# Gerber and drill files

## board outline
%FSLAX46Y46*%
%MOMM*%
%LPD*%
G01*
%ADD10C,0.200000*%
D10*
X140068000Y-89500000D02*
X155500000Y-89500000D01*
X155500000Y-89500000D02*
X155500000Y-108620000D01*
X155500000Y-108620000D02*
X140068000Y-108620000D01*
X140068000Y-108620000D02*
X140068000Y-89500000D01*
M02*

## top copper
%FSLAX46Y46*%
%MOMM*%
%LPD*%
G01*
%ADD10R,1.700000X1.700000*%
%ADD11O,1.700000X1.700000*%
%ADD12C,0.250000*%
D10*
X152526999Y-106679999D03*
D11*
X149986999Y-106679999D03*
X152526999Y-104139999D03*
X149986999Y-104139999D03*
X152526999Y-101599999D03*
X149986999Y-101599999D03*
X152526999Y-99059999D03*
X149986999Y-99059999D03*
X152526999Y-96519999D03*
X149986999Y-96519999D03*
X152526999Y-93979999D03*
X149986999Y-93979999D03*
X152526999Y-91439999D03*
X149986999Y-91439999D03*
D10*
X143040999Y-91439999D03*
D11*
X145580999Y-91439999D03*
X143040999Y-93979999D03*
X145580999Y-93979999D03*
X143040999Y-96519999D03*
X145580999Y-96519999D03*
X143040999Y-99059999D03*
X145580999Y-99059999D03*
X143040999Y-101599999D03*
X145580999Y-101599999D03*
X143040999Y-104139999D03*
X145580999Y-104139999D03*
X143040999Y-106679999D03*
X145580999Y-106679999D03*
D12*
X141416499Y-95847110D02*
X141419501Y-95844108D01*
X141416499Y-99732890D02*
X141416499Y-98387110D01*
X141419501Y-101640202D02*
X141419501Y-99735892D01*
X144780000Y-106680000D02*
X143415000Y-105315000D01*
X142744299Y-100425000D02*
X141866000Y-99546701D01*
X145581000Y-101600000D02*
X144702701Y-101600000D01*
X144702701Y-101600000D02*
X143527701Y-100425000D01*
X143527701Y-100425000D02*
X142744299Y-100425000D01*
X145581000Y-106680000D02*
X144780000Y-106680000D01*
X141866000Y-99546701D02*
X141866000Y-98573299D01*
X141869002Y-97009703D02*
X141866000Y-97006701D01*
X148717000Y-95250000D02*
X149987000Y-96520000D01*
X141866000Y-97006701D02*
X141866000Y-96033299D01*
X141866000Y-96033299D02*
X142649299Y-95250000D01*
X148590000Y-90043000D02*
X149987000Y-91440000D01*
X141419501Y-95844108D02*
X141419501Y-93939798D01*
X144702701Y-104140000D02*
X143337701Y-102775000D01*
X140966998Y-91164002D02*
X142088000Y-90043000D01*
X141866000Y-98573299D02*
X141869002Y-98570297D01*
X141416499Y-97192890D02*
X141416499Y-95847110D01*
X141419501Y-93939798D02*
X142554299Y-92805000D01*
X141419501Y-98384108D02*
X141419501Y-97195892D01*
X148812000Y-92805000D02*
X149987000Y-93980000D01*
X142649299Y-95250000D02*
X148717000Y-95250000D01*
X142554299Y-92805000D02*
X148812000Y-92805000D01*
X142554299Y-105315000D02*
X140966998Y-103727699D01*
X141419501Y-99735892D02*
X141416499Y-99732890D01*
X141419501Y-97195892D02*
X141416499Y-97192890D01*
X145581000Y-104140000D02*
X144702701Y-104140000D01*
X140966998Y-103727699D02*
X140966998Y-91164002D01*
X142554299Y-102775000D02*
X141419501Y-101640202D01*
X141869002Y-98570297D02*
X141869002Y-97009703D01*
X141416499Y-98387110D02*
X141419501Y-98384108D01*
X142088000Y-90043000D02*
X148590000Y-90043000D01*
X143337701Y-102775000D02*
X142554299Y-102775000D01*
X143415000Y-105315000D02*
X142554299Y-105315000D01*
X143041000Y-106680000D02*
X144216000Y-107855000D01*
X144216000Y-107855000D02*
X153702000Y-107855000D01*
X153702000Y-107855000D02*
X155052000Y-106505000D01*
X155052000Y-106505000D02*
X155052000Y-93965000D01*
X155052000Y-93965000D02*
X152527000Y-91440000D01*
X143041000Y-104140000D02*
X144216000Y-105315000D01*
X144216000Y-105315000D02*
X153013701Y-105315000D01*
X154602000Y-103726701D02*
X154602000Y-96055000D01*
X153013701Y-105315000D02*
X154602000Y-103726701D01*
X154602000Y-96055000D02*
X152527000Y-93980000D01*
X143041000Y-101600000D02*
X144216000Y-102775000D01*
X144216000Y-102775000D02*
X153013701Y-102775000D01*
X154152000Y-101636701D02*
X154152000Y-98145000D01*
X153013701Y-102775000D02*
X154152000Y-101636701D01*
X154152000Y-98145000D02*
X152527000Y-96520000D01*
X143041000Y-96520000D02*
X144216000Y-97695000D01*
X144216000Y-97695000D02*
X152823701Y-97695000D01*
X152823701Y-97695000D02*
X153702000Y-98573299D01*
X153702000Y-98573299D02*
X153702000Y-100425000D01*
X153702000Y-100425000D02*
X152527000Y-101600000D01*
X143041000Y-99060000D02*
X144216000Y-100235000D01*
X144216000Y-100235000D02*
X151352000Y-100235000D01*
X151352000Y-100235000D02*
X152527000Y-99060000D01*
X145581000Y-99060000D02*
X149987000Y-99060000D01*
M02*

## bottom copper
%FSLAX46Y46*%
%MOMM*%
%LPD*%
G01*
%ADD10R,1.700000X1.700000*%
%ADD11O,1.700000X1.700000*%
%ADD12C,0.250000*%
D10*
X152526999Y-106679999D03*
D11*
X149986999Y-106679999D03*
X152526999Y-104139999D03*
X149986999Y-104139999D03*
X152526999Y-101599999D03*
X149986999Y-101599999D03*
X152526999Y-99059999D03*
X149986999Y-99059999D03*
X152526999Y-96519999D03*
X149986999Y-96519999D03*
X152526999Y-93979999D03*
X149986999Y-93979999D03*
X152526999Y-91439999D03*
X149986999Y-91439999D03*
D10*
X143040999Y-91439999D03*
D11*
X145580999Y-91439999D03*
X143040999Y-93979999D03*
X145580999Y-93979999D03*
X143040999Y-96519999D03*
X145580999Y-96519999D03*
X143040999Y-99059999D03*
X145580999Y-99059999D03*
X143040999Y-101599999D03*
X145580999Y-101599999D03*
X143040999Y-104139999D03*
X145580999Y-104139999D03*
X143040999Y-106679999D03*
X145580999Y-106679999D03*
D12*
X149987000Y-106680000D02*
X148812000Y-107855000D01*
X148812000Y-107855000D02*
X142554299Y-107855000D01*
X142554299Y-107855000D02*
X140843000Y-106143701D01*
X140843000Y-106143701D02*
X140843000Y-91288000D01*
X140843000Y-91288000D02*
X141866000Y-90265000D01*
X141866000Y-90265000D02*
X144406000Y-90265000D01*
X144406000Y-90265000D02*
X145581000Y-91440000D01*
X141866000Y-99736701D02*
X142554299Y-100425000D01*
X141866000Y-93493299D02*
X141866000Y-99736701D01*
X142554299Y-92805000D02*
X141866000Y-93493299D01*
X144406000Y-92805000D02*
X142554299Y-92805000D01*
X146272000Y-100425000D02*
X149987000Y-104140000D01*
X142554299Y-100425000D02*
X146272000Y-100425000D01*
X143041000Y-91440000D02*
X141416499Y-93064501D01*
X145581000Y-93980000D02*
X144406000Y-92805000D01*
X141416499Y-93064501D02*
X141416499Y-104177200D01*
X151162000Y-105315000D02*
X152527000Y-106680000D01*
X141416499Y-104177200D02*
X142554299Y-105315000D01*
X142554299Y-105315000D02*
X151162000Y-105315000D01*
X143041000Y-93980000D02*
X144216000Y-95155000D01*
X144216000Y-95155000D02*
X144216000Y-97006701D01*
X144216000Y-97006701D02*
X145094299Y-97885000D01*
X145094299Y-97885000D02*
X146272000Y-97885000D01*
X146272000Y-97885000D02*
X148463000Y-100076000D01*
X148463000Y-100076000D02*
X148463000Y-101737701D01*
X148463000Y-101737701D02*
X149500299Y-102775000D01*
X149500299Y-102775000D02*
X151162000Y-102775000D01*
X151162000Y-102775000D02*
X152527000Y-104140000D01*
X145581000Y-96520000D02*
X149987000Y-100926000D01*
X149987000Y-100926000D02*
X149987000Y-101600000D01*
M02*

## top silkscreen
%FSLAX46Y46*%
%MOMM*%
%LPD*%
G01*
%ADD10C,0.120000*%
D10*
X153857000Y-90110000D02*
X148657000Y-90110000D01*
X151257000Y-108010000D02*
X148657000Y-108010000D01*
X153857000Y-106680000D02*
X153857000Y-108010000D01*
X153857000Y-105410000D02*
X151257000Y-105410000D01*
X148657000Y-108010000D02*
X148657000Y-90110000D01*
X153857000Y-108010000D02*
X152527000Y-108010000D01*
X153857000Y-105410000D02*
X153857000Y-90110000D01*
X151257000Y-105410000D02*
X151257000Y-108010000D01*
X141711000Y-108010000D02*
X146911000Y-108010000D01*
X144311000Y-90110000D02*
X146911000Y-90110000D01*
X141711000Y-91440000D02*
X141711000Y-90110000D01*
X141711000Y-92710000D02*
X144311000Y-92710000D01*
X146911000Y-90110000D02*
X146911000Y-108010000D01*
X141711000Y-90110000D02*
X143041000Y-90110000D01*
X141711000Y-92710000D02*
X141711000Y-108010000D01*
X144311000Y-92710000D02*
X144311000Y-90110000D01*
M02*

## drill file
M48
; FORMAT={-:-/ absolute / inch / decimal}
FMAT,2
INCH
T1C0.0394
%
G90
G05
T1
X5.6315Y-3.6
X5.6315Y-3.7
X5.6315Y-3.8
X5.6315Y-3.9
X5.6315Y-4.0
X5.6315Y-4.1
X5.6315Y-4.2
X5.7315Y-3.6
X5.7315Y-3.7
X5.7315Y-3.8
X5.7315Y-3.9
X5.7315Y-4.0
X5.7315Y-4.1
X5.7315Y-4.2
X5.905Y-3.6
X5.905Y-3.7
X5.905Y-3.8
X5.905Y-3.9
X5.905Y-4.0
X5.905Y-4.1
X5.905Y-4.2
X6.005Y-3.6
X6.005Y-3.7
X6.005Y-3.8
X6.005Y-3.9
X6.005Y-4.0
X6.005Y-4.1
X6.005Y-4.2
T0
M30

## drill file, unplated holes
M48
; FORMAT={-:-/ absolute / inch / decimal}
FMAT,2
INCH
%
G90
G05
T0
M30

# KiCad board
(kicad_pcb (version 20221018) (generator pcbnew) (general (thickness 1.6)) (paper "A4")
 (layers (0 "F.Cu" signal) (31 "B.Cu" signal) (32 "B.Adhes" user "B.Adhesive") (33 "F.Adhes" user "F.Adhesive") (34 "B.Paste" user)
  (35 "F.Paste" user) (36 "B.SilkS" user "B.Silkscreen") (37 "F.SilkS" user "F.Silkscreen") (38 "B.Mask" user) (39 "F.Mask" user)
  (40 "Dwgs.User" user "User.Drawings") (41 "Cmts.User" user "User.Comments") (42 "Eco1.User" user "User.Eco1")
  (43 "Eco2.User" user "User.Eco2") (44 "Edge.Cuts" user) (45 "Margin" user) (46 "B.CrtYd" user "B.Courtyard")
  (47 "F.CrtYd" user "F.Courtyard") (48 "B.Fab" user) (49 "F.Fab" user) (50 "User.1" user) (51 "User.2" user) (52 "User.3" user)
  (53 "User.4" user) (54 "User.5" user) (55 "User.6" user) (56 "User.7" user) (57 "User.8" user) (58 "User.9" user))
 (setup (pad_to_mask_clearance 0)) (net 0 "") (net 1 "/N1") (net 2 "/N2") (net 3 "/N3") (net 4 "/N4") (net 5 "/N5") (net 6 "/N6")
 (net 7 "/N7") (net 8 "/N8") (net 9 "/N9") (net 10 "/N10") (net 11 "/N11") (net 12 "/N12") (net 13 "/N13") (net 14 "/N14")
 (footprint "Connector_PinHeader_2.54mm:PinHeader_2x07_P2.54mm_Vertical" (layer "F.Cu") (at 143.041 91.44)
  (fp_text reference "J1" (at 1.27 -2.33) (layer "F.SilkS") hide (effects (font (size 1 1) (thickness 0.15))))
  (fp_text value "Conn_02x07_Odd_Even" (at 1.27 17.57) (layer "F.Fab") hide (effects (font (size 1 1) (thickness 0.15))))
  (fp_line (start -1.33 -1.33) (end 0 -1.33) (stroke (width 0.12) (type solid)) (layer "F.SilkS"))
  (fp_line (start -1.33 0) (end -1.33 -1.33) (stroke (width 0.12) (type solid)) (layer "F.SilkS"))
  (fp_line (start -1.33 1.27) (end -1.33 16.57) (stroke (width 0.12) (type solid)) (layer "F.SilkS"))
  (fp_line (start -1.33 1.27) (end 1.27 1.27) (stroke (width 0.12) (type solid)) (layer "F.SilkS"))
  (fp_line (start -1.33 16.57) (end 3.87 16.57) (stroke (width 0.12) (type solid)) (layer "F.SilkS"))
  (fp_line (start 1.27 -1.33) (end 3.87 -1.33) (stroke (width 0.12) (type solid)) (layer "F.SilkS"))
  (fp_line (start 1.27 1.27) (end 1.27 -1.33) (stroke (width 0.12) (type solid)) (layer "F.SilkS"))
  (fp_line (start 3.87 -1.33) (end 3.87 16.57) (stroke (width 0.12) (type solid)) (layer "F.SilkS"))
  (pad "1" thru_hole rect (at 0 0) (size 1.7 1.7) (drill 1) (layers "*.Cu" "*.Mask") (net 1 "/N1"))
  (pad "2" thru_hole oval (at 2.54 0) (size 1.7 1.7) (drill 1) (layers "*.Cu" "*.Mask") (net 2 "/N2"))
  (pad "3" thru_hole oval (at 0 2.54) (size 1.7 1.7) (drill 1) (layers "*.Cu" "*.Mask") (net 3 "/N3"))
  (pad "4" thru_hole oval (at 2.54 2.54) (size 1.7 1.7) (drill 1) (layers "*.Cu" "*.Mask") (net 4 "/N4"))
  (pad "5" thru_hole oval (at 0 5.08) (size 1.7 1.7) (drill 1) (layers "*.Cu" "*.Mask") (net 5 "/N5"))
  (pad "6" thru_hole oval (at 2.54 5.08) (size 1.7 1.7) (drill 1) (layers "*.Cu" "*.Mask") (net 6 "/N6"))
  (pad "7" thru_hole oval (at 0 7.62) (size 1.7 1.7) (drill 1) (layers "*.Cu" "*.Mask") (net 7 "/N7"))
  (pad "8" thru_hole oval (at 2.54 7.62) (size 1.7 1.7) (drill 1) (layers "*.Cu" "*.Mask") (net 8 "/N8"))
  (pad "9" thru_hole oval (at 0 10.16) (size 1.7 1.7) (drill 1) (layers "*.Cu" "*.Mask") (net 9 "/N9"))
  (pad "10" thru_hole oval (at 2.54 10.16) (size 1.7 1.7) (drill 1) (layers "*.Cu" "*.Mask") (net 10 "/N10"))
  (pad "11" thru_hole oval (at 0 12.7) (size 1.7 1.7) (drill 1) (layers "*.Cu" "*.Mask") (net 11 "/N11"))
  (pad "12" thru_hole oval (at 2.54 12.7) (size 1.7 1.7) (drill 1) (layers "*.Cu" "*.Mask") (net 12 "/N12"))
  (pad "13" thru_hole oval (at 0 15.24) (size 1.7 1.7) (drill 1) (layers "*.Cu" "*.Mask") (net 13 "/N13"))
  (pad "14" thru_hole oval (at 2.54 15.24) (size 1.7 1.7) (drill 1) (layers "*.Cu" "*.Mask") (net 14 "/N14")))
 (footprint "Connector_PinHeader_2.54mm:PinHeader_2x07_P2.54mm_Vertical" (layer "F.Cu") (at 152.527 106.68 180)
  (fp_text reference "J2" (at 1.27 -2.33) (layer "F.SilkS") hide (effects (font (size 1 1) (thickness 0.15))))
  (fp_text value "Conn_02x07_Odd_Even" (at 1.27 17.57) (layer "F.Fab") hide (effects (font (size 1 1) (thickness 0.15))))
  (fp_line (start -1.33 -1.33) (end 0 -1.33) (stroke (width 0.12) (type solid)) (layer "F.SilkS"))
  (fp_line (start -1.33 0) (end -1.33 -1.33) (stroke (width 0.12) (type solid)) (layer "F.SilkS"))
  (fp_line (start -1.33 1.27) (end -1.33 16.57) (stroke (width 0.12) (type solid)) (layer "F.SilkS"))
  (fp_line (start -1.33 1.27) (end 1.27 1.27) (stroke (width 0.12) (type solid)) (layer "F.SilkS"))
  (fp_line (start -1.33 16.57) (end 3.87 16.57) (stroke (width 0.12) (type solid)) (layer "F.SilkS"))
  (fp_line (start 1.27 -1.33) (end 3.87 -1.33) (stroke (width 0.12) (type solid)) (layer "F.SilkS"))
  (fp_line (start 1.27 1.27) (end 1.27 -1.33) (stroke (width 0.12) (type solid)) (layer "F.SilkS"))
  (fp_line (start 3.87 -1.33) (end 3.87 16.57) (stroke (width 0.12) (type solid)) (layer "F.SilkS"))
  (pad "1" thru_hole rect (at 0 0 180) (size 1.7 1.7) (drill 1) (layers "*.Cu" "*.Mask") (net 1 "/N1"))
  (pad "2" thru_hole oval (at 2.54 0 180) (size 1.7 1.7) (drill 1) (layers "*.Cu" "*.Mask") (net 2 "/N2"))
  (pad "3" thru_hole oval (at 0 2.54 180) (size 1.7 1.7) (drill 1) (layers "*.Cu" "*.Mask") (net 3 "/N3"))
  (pad "4" thru_hole oval (at 2.54 2.54 180) (size 1.7 1.7) (drill 1) (layers "*.Cu" "*.Mask") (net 4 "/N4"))
  (pad "5" thru_hole oval (at 0 5.08 180) (size 1.7 1.7) (drill 1) (layers "*.Cu" "*.Mask") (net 5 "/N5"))
  (pad "6" thru_hole oval (at 2.54 5.08 180) (size 1.7 1.7) (drill 1) (layers "*.Cu" "*.Mask") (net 6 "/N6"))
  (pad "7" thru_hole oval (at 0 7.62 180) (size 1.7 1.7) (drill 1) (layers "*.Cu" "*.Mask") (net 7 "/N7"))
  (pad "8" thru_hole oval (at 2.54 7.62 180) (size 1.7 1.7) (drill 1) (layers "*.Cu" "*.Mask") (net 8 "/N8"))
  (pad "9" thru_hole oval (at 0 10.16 180) (size 1.7 1.7) (drill 1) (layers "*.Cu" "*.Mask") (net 9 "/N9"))
  (pad "10" thru_hole oval (at 2.54 10.16 180) (size 1.7 1.7) (drill 1) (layers "*.Cu" "*.Mask") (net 10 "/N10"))
  (pad "11" thru_hole oval (at 0 12.7 180) (size 1.7 1.7) (drill 1) (layers "*.Cu" "*.Mask") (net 11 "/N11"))
  (pad "12" thru_hole oval (at 2.54 12.7 180) (size 1.7 1.7) (drill 1) (layers "*.Cu" "*.Mask") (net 12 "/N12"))
  (pad "13" thru_hole oval (at 0 15.24 180) (size 1.7 1.7) (drill 1) (layers "*.Cu" "*.Mask") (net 13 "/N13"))
  (pad "14" thru_hole oval (at 2.54 15.24 180) (size 1.7 1.7) (drill 1) (layers "*.Cu" "*.Mask") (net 14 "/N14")))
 (gr_rect (start 140.068 89.5) (end 155.5 108.62) (stroke (width 0.2) (type default)) (fill none) (layer "Edge.Cuts"))
 (segment (start 142.554299 105.315) (end 151.162 105.315) (width 0.25) (layer "B.Cu") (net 1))
 (segment (start 143.041 91.44) (end 141.416499 93.064501) (width 0.25) (layer "B.Cu") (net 1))
 (segment (start 151.162 105.315) (end 152.527 106.68) (width 0.25) (layer "B.Cu") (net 1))
 (segment (start 141.416499 93.064501) (end 141.416499 104.1772) (width 0.25) (layer "B.Cu") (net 1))
 (segment (start 141.416499 104.1772) (end 142.554299 105.315) (width 0.25) (layer "B.Cu") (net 1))
 (segment (start 149.987 106.68) (end 148.812 107.855) (width 0.25) (layer "B.Cu") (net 2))
 (segment (start 148.812 107.855) (end 142.554299 107.855) (width 0.25) (layer "B.Cu") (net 2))
 (segment (start 140.843 91.288) (end 141.866 90.265) (width 0.25) (layer "B.Cu") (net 2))
 (segment (start 144.406 90.265) (end 145.581 91.44) (width 0.25) (layer "B.Cu") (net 2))
 (segment (start 142.554299 107.855) (end 140.843 106.143701) (width 0.25) (layer "B.Cu") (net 2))
 (segment (start 140.843 106.143701) (end 140.843 91.288) (width 0.25) (layer "B.Cu") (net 2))
 (segment (start 141.866 90.265) (end 144.406 90.265) (width 0.25) (layer "B.Cu") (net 2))
 (segment (start 148.463 100.076) (end 148.463 101.737701) (width 0.25) (layer "B.Cu") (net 3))
 (segment (start 151.162 102.775) (end 152.527 104.14) (width 0.25) (layer "B.Cu") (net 3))
 (segment (start 143.041 93.98) (end 144.216 95.155) (width 0.25) (layer "B.Cu") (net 3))
 (segment (start 145.094299 97.885) (end 146.272 97.885) (width 0.25) (layer "B.Cu") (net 3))
 (segment (start 144.216 95.155) (end 144.216 97.006701) (width 0.25) (layer "B.Cu") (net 3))
 (segment (start 149.500299 102.775) (end 151.162 102.775) (width 0.25) (layer "B.Cu") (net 3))
 (segment (start 148.463 101.737701) (end 149.500299 102.775) (width 0.25) (layer "B.Cu") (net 3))
 (segment (start 144.216 97.006701) (end 145.094299 97.885) (width 0.25) (layer "B.Cu") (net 3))
 (segment (start 146.272 97.885) (end 148.463 100.076) (width 0.25) (layer "B.Cu") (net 3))
 (segment (start 145.581 93.98) (end 144.406 92.805) (width 0.25) (layer "B.Cu") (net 4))
 (segment (start 142.554299 100.425) (end 146.272 100.425) (width 0.25) (layer "B.Cu") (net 4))
 (segment (start 144.406 92.805) (end 142.554299 92.805) (width 0.25) (layer "B.Cu") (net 4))
 (segment (start 141.866 99.736701) (end 142.554299 100.425) (width 0.25) (layer "B.Cu") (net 4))
 (segment (start 142.554299 92.805) (end 141.866 93.493299) (width 0.25) (layer "B.Cu") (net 4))
 (segment (start 141.866 93.493299) (end 141.866 99.736701) (width 0.25) (layer "B.Cu") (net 4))
 (segment (start 146.272 100.425) (end 149.987 104.14) (width 0.25) (layer "B.Cu") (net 4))
 (segment (start 143.041 96.52) (end 144.216 97.695) (width 0.25) (layer "F.Cu") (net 5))
 (segment (start 144.216 97.695) (end 152.823701 97.695) (width 0.25) (layer "F.Cu") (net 5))
 (segment (start 153.702 98.573299) (end 153.702 100.425) (width 0.25) (layer "F.Cu") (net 5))
 (segment (start 153.702 100.425) (end 152.527 101.6) (width 0.25) (layer "F.Cu") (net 5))
 (segment (start 152.823701 97.695) (end 153.702 98.573299) (width 0.25) (layer "F.Cu") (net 5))
 (segment (start 145.581 96.52) (end 149.987 100.926) (width 0.25) (layer "B.Cu") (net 6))
 (segment (start 149.987 100.926) (end 149.987 101.6) (width 0.25) (layer "B.Cu") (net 6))
 (segment (start 143.041 99.06) (end 144.216 100.235) (width 0.25) (layer "F.Cu") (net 7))
 (segment (start 144.216 100.235) (end 151.352 100.235) (width 0.25) (layer "F.Cu") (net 7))
 (segment (start 151.352 100.235) (end 152.527 99.06) (width 0.25) (layer "F.Cu") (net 7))
 (segment (start 145.581 99.06) (end 149.987 99.06) (width 0.25) (layer "F.Cu") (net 8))
 (segment (start 154.152 101.636701) (end 154.152 98.145) (width 0.25) (layer "F.Cu") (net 9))
 (segment (start 144.216 102.775) (end 153.013701 102.775) (width 0.25) (layer "F.Cu") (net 9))
 (segment (start 143.041 101.6) (end 144.216 102.775) (width 0.25) (layer "F.Cu") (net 9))
 (segment (start 154.152 98.145) (end 152.527 96.52) (width 0.25) (layer "F.Cu") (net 9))
 (segment (start 153.013701 102.775) (end 154.152 101.636701) (width 0.25) (layer "F.Cu") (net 9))
 (segment (start 141.866 96.033299) (end 142.649299 95.25) (width 0.25) (layer "F.Cu") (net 10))
 (segment (start 141.866 99.546701) (end 141.866 98.573299) (width 0.25) (layer "F.Cu") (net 10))
 (segment (start 141.866 98.573299) (end 141.869002 98.570297) (width 0.25) (layer "F.Cu") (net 10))
 (segment (start 144.702701 101.6) (end 143.527701 100.425) (width 0.25) (layer "F.Cu") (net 10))
 (segment (start 141.869002 98.570297) (end 141.869002 97.009703) (width 0.25) (layer "F.Cu") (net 10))
 (segment (start 143.527701 100.425) (end 142.744299 100.425) (width 0.25) (layer "F.Cu") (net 10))
 (segment (start 145.581 101.6) (end 144.702701 101.6) (width 0.25) (layer "F.Cu") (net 10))
 (segment (start 142.744299 100.425) (end 141.866 99.546701) (width 0.25) (layer "F.Cu") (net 10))
 (segment (start 142.649299 95.25) (end 148.717 95.25) (width 0.25) (layer "F.Cu") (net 10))
 (segment (start 141.866 97.006701) (end 141.866 96.033299) (width 0.25) (layer "F.Cu") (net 10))
 (segment (start 148.717 95.25) (end 149.987 96.52) (width 0.25) (layer "F.Cu") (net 10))
 (segment (start 141.869002 97.009703) (end 141.866 97.006701) (width 0.25) (layer "F.Cu") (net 10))
 (segment (start 144.216 105.315) (end 153.013701 105.315) (width 0.25) (layer "F.Cu") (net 11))
 (segment (start 153.013701 105.315) (end 154.602 103.726701) (width 0.25) (layer "F.Cu") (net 11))
 (segment (start 143.041 104.14) (end 144.216 105.315) (width 0.25) (layer "F.Cu") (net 11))
 (segment (start 154.602 96.055) (end 152.527 93.98) (width 0.25) (layer "F.Cu") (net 11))
 (segment (start 154.602 103.726701) (end 154.602 96.055) (width 0.25) (layer "F.Cu") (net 11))
 (segment (start 141.416499 95.84711) (end 141.419501 95.844108) (width 0.25) (layer "F.Cu") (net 12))
 (segment (start 141.419501 93.939798) (end 142.554299 92.805) (width 0.25) (layer "F.Cu") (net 12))
 (segment (start 141.419501 98.384108) (end 141.419501 97.195892) (width 0.25) (layer "F.Cu") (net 12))
 (segment (start 141.419501 95.844108) (end 141.419501 93.939798) (width 0.25) (layer "F.Cu") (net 12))
 (segment (start 141.419501 97.195892) (end 141.416499 97.19289) (width 0.25) (layer "F.Cu") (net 12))
 (segment (start 142.554299 92.805) (end 148.812 92.805) (width 0.25) (layer "F.Cu") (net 12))
 (segment (start 148.812 92.805) (end 149.987 93.98) (width 0.25) (layer "F.Cu") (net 12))
 (segment (start 145.581 104.14) (end 144.702701 104.14) (width 0.25) (layer "F.Cu") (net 12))
 (segment (start 141.419501 99.735892) (end 141.416499 99.73289) (width 0.25) (layer "F.Cu") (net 12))
 (segment (start 141.416499 98.38711) (end 141.419501 98.384108) (width 0.25) (layer "F.Cu") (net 12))
 (segment (start 141.416499 97.19289) (end 141.416499 95.84711) (width 0.25) (layer "F.Cu") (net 12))
 (segment (start 144.702701 104.14) (end 143.337701 102.775) (width 0.25) (layer "F.Cu") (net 12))
 (segment (start 142.554299 102.775) (end 141.419501 101.640202) (width 0.25) (layer "F.Cu") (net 12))
 (segment (start 141.419501 101.640202) (end 141.419501 99.735892) (width 0.25) (layer "F.Cu") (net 12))
 (segment (start 143.337701 102.775) (end 142.554299 102.775) (width 0.25) (layer "F.Cu") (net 12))
 (segment (start 141.416499 99.73289) (end 141.416499 98.38711) (width 0.25) (layer "F.Cu") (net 12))
 (segment (start 143.041 106.68) (end 144.216 107.855) (width 0.25) (layer "F.Cu") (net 13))
 (segment (start 155.052 106.505) (end 155.052 93.965) (width 0.25) (layer "F.Cu") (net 13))
 (segment (start 155.052 93.965) (end 152.527 91.44) (width 0.25) (layer "F.Cu") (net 13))
 (segment (start 153.702 107.855) (end 155.052 106.505) (width 0.25) (layer "F.Cu") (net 13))
 (segment (start 144.216 107.855) (end 153.702 107.855) (width 0.25) (layer "F.Cu") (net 13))
 (segment (start 148.59 90.043) (end 149.987 91.44) (width 0.25) (layer "F.Cu") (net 14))
 (segment (start 142.088 90.043) (end 148.59 90.043) (width 0.25) (layer "F.Cu") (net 14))
 (segment (start 142.554299 105.315) (end 140.966998 103.727699) (width 0.25) (layer "F.Cu") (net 14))
 (segment (start 140.966998 103.727699) (end 140.966998 91.164002) (width 0.25) (layer "F.Cu") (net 14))
 (segment (start 145.581 106.68) (end 144.78 106.68) (width 0.25) (layer "F.Cu") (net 14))
 (segment (start 144.78 106.68) (end 143.415 105.315) (width 0.25) (layer "F.Cu") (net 14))
 (segment (start 140.966998 91.164002) (end 142.088 90.043) (width 0.25) (layer "F.Cu") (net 14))
 (segment (start 143.415 105.315) (end 142.554299 105.315) (width 0.25) (layer "F.Cu") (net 14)))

